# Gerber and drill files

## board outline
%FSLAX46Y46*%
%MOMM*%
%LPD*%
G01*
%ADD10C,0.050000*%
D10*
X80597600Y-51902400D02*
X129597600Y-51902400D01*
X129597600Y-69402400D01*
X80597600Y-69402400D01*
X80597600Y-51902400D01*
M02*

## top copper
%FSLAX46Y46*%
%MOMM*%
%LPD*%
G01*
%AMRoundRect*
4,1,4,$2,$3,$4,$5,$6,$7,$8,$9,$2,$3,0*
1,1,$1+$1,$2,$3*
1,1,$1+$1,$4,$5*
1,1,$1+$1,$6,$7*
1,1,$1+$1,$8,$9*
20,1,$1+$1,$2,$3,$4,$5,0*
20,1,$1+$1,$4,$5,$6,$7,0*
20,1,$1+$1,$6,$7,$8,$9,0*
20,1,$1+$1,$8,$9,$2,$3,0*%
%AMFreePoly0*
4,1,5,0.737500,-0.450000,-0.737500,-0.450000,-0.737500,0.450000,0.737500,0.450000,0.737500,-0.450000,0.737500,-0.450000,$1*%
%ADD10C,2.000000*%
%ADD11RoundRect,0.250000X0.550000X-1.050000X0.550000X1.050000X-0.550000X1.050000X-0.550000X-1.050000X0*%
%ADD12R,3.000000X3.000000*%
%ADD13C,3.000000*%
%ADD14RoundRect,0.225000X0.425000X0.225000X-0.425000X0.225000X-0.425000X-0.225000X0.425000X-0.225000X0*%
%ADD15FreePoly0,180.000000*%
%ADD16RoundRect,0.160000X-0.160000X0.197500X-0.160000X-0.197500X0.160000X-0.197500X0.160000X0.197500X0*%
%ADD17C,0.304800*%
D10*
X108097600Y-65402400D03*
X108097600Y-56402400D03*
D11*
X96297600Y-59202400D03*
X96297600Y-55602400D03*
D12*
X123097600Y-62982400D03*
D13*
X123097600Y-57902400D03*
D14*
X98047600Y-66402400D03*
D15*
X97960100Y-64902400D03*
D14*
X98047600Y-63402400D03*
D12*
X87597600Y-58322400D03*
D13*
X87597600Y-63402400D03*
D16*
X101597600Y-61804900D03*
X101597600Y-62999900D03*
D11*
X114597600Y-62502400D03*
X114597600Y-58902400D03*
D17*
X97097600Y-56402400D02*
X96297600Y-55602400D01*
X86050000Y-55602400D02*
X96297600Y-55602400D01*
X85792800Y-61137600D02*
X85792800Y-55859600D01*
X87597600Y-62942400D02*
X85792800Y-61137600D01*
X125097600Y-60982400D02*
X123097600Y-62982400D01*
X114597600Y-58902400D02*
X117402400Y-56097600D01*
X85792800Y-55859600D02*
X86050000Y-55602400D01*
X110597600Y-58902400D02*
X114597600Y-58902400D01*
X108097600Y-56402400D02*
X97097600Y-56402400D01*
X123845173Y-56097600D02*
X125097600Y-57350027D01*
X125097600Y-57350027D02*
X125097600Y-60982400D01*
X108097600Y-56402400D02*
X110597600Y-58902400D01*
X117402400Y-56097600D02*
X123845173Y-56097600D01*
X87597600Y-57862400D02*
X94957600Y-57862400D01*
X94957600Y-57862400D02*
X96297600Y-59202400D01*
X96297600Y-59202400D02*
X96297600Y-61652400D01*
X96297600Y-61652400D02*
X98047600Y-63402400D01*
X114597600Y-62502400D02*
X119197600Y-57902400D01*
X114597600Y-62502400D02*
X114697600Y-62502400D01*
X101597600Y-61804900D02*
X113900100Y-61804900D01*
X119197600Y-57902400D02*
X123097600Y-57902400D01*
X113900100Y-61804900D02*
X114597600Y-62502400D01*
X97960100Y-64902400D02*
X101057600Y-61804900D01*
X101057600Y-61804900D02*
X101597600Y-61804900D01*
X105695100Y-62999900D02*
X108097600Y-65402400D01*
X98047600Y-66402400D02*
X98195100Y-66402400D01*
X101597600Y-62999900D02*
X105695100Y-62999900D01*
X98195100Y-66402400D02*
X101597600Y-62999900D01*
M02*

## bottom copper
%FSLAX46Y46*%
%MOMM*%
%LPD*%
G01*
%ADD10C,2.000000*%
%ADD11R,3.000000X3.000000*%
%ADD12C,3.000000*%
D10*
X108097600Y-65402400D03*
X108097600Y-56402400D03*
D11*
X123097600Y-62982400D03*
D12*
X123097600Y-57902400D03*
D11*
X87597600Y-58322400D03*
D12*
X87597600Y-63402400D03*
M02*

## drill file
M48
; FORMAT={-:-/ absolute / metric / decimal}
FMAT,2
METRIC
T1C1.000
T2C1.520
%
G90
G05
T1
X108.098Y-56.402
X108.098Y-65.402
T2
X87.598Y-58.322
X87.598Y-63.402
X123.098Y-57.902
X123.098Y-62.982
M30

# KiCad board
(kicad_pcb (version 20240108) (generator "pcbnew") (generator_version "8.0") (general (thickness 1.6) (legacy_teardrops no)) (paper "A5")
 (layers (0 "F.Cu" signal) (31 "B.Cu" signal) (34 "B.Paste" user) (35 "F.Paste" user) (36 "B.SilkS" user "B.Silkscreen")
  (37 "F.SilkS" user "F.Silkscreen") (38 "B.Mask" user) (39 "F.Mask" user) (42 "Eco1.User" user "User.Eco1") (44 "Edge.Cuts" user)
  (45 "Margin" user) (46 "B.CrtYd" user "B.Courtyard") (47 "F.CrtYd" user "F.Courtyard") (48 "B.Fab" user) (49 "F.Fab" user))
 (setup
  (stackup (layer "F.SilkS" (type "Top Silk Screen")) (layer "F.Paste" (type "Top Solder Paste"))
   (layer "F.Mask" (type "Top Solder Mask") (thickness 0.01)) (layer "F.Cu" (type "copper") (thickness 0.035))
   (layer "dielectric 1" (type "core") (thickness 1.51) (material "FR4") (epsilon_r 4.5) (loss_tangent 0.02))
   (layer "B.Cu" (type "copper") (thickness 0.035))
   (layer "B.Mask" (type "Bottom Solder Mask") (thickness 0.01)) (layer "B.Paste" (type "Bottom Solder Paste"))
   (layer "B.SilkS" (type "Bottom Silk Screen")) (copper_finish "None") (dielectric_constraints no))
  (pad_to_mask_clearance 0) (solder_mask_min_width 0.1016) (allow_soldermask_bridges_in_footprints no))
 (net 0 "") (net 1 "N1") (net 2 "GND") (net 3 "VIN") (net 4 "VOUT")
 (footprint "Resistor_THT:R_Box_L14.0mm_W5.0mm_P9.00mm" (layer "F.Cu") (at 108.0976 65.4024 90)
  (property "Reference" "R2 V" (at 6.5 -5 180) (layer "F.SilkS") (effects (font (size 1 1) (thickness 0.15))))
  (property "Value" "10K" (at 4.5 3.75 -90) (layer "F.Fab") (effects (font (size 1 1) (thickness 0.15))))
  (pad "1" thru_hole circle (at 0 0 90) (size 2 2) (drill 1) (layers "*.Cu" "*.Mask") (remove_unused_layers no) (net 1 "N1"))
  (pad "2" thru_hole circle (at 9 0 90) (size 2 2) (drill 1) (layers "*.Cu" "*.Mask") (remove_unused_layers no) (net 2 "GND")))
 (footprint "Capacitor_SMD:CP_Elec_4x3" (layer "F.Cu") (at 96.2976 57.4024 90)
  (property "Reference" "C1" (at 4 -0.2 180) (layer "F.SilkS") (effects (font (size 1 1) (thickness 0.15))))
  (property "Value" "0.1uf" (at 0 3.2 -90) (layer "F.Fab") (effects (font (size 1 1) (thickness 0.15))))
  (pad "1" smd roundrect (at -1.8 0 90) (size 2.6 1.6) (layers "F.Cu" "F.Paste" "F.Mask") (roundrect_rratio 0.15625) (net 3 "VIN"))
  (pad "2" smd roundrect (at 1.8 0 90) (size 2.6 1.6) (layers "F.Cu" "F.Paste" "F.Mask") (roundrect_rratio 0.15625) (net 2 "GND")))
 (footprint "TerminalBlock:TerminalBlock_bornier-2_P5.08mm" (layer "F.Cu") (at 123.0976 62.9824 90)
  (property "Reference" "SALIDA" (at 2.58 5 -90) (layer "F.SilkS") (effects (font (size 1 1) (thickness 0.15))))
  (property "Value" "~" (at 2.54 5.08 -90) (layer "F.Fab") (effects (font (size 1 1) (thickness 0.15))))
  (pad "1" thru_hole rect (at 0 0 90) (size 3 3) (drill 1.52) (layers "*.Cu" "*.Mask") (remove_unused_layers no) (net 2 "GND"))
  (pad "2" thru_hole circle (at 5.08 0 90) (size 3 3) (drill 1.52) (layers "*.Cu" "*.Mask") (remove_unused_layers no) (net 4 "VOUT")))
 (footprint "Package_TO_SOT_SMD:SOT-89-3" (layer "F.Cu") (at 96.0976 64.9024 180)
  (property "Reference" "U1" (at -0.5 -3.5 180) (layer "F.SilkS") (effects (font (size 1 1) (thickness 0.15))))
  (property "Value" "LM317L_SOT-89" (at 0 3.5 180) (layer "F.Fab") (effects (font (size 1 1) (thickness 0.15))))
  (pad "1" smd roundrect (at -1.95 -1.5 180) (size 1.3 0.9) (layers "F.Cu" "F.Paste" "F.Mask") (roundrect_rratio 0.25) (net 1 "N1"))
  (pad "2" smd custom (at -1.8625 0 180) (size 1.475 0.9) (layers "F.Cu" "F.Paste" "F.Mask") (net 4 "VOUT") (zone_connect 2)
   (thermal_bridge_angle 45) (options (clearance outline) (anchor rect)) (primitives))
  (pad "3" smd roundrect (at -1.95 1.5 180) (size 1.3 0.9) (layers "F.Cu" "F.Paste" "F.Mask") (roundrect_rratio 0.25) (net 3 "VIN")))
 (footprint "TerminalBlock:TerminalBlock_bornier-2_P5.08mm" (layer "F.Cu") (at 87.5976 58.3224 -90)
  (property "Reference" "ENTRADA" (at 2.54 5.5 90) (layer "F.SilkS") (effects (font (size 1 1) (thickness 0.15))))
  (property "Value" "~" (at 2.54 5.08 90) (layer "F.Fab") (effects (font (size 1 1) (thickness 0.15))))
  (pad "1" thru_hole rect (at 0 0 270) (size 3 3) (drill 1.52) (layers "*.Cu" "*.Mask") (remove_unused_layers no) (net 3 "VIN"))
  (pad "2" thru_hole circle (at 5.08 0 270) (size 3 3) (drill 1.52) (layers "*.Cu" "*.Mask") (remove_unused_layers no) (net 2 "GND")))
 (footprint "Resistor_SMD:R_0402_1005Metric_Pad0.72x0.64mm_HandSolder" (layer "F.Cu") (at 101.5976 62.4024 -90)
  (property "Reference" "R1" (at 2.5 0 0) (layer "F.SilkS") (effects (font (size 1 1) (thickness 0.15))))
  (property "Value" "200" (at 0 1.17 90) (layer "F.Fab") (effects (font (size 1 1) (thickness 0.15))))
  (pad "1" smd roundrect (at -0.5975 0 270) (size 0.715 0.64) (layers "F.Cu" "F.Paste" "F.Mask") (roundrect_rratio 0.25) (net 4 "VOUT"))
  (pad "2" smd roundrect (at 0.5975 0 270) (size 0.715 0.64) (layers "F.Cu" "F.Paste" "F.Mask") (roundrect_rratio 0.25) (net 1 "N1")))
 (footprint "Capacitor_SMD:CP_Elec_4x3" (layer "F.Cu") (at 114.5976 60.7024 90)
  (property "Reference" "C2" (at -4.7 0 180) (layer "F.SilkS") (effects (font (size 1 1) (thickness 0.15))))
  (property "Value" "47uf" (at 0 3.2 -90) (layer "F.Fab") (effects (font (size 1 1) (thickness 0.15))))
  (pad "1" smd roundrect (at -1.8 0 90) (size 2.6 1.6) (layers "F.Cu" "F.Paste" "F.Mask") (roundrect_rratio 0.15625) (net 4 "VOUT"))
  (pad "2" smd roundrect (at 1.8 0 90) (size 2.6 1.6) (layers "F.Cu" "F.Paste" "F.Mask") (roundrect_rratio 0.15625) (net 2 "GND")))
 (gr_rect (start 80.5976 51.9024) (end 129.5976 69.4024) (stroke (width 0.05) (type default)) (fill none) (layer "Edge.Cuts"))
 (segment (start 97.0976 56.4024) (end 96.2976 55.6024) (width 0.3048) (layer "F.Cu") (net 2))
 (segment (start 86.05 55.6024) (end 96.2976 55.6024) (width 0.3048) (layer "F.Cu") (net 2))
 (segment (start 85.7928 61.1376) (end 85.7928 55.8596) (width 0.3048) (layer "F.Cu") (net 2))
 (segment (start 87.5976 62.9424) (end 85.7928 61.1376) (width 0.3048) (layer "F.Cu") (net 2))
 (segment (start 125.0976 60.9824) (end 123.0976 62.9824) (width 0.3048) (layer "F.Cu") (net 2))
 (segment (start 114.5976 58.9024) (end 117.4024 56.0976) (width 0.3048) (layer "F.Cu") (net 2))
 (segment (start 85.7928 55.8596) (end 86.05 55.6024) (width 0.3048) (layer "F.Cu") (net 2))
 (segment (start 110.5976 58.9024) (end 114.5976 58.9024) (width 0.3048) (layer "F.Cu") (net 2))
 (segment (start 108.0976 56.4024) (end 97.0976 56.4024) (width 0.3048) (layer "F.Cu") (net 2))
 (segment (start 123.845173 56.0976) (end 125.0976 57.350027) (width 0.3048) (layer "F.Cu") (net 2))
 (segment (start 125.0976 57.350027) (end 125.0976 60.9824) (width 0.3048) (layer "F.Cu") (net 2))
 (segment (start 108.0976 56.4024) (end 110.5976 58.9024) (width 0.3048) (layer "F.Cu") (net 2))
 (segment (start 117.4024 56.0976) (end 123.845173 56.0976) (width 0.3048) (layer "F.Cu") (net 2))
 (segment (start 87.5976 57.8624) (end 94.9576 57.8624) (width 0.3048) (layer "F.Cu") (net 3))
 (segment (start 94.9576 57.8624) (end 96.2976 59.2024) (width 0.3048) (layer "F.Cu") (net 3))
 (segment (start 96.2976 59.2024) (end 96.2976 61.6524) (width 0.3048) (layer "F.Cu") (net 3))
 (segment (start 96.2976 61.6524) (end 98.0476 63.4024) (width 0.3048) (layer "F.Cu") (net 3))
 (segment (start 114.5976 62.5024) (end 119.1976 57.9024) (width 0.3048) (layer "F.Cu") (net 4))
 (segment (start 114.5976 62.5024) (end 114.6976 62.5024) (width 0.3048) (layer "F.Cu") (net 4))
 (segment (start 101.5976 61.8049) (end 113.9001 61.8049) (width 0.3048) (layer "F.Cu") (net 4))
 (segment (start 119.1976 57.9024) (end 123.0976 57.9024) (width 0.3048) (layer "F.Cu") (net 4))
 (segment (start 113.9001 61.8049) (end 114.5976 62.5024) (width 0.3048) (layer "F.Cu") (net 4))
 (segment (start 97.9601 64.9024) (end 101.0576 61.8049) (width 0.3048) (layer "F.Cu") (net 4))
 (segment (start 101.0576 61.8049) (end 101.5976 61.8049) (width 0.3048) (layer "F.Cu") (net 4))
 (segment (start 105.6951 62.9999) (end 108.0976 65.4024) (width 0.3048) (layer "F.Cu") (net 1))
 (segment (start 98.0476 66.4024) (end 98.1951 66.4024) (width 0.3048) (layer "F.Cu") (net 1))
 (segment (start 101.5976 62.9999) (end 105.6951 62.9999) (width 0.3048) (layer "F.Cu") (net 1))
 (segment (start 98.1951 66.4024) (end 101.5976 62.9999) (width 0.3048) (layer "F.Cu") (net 1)))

